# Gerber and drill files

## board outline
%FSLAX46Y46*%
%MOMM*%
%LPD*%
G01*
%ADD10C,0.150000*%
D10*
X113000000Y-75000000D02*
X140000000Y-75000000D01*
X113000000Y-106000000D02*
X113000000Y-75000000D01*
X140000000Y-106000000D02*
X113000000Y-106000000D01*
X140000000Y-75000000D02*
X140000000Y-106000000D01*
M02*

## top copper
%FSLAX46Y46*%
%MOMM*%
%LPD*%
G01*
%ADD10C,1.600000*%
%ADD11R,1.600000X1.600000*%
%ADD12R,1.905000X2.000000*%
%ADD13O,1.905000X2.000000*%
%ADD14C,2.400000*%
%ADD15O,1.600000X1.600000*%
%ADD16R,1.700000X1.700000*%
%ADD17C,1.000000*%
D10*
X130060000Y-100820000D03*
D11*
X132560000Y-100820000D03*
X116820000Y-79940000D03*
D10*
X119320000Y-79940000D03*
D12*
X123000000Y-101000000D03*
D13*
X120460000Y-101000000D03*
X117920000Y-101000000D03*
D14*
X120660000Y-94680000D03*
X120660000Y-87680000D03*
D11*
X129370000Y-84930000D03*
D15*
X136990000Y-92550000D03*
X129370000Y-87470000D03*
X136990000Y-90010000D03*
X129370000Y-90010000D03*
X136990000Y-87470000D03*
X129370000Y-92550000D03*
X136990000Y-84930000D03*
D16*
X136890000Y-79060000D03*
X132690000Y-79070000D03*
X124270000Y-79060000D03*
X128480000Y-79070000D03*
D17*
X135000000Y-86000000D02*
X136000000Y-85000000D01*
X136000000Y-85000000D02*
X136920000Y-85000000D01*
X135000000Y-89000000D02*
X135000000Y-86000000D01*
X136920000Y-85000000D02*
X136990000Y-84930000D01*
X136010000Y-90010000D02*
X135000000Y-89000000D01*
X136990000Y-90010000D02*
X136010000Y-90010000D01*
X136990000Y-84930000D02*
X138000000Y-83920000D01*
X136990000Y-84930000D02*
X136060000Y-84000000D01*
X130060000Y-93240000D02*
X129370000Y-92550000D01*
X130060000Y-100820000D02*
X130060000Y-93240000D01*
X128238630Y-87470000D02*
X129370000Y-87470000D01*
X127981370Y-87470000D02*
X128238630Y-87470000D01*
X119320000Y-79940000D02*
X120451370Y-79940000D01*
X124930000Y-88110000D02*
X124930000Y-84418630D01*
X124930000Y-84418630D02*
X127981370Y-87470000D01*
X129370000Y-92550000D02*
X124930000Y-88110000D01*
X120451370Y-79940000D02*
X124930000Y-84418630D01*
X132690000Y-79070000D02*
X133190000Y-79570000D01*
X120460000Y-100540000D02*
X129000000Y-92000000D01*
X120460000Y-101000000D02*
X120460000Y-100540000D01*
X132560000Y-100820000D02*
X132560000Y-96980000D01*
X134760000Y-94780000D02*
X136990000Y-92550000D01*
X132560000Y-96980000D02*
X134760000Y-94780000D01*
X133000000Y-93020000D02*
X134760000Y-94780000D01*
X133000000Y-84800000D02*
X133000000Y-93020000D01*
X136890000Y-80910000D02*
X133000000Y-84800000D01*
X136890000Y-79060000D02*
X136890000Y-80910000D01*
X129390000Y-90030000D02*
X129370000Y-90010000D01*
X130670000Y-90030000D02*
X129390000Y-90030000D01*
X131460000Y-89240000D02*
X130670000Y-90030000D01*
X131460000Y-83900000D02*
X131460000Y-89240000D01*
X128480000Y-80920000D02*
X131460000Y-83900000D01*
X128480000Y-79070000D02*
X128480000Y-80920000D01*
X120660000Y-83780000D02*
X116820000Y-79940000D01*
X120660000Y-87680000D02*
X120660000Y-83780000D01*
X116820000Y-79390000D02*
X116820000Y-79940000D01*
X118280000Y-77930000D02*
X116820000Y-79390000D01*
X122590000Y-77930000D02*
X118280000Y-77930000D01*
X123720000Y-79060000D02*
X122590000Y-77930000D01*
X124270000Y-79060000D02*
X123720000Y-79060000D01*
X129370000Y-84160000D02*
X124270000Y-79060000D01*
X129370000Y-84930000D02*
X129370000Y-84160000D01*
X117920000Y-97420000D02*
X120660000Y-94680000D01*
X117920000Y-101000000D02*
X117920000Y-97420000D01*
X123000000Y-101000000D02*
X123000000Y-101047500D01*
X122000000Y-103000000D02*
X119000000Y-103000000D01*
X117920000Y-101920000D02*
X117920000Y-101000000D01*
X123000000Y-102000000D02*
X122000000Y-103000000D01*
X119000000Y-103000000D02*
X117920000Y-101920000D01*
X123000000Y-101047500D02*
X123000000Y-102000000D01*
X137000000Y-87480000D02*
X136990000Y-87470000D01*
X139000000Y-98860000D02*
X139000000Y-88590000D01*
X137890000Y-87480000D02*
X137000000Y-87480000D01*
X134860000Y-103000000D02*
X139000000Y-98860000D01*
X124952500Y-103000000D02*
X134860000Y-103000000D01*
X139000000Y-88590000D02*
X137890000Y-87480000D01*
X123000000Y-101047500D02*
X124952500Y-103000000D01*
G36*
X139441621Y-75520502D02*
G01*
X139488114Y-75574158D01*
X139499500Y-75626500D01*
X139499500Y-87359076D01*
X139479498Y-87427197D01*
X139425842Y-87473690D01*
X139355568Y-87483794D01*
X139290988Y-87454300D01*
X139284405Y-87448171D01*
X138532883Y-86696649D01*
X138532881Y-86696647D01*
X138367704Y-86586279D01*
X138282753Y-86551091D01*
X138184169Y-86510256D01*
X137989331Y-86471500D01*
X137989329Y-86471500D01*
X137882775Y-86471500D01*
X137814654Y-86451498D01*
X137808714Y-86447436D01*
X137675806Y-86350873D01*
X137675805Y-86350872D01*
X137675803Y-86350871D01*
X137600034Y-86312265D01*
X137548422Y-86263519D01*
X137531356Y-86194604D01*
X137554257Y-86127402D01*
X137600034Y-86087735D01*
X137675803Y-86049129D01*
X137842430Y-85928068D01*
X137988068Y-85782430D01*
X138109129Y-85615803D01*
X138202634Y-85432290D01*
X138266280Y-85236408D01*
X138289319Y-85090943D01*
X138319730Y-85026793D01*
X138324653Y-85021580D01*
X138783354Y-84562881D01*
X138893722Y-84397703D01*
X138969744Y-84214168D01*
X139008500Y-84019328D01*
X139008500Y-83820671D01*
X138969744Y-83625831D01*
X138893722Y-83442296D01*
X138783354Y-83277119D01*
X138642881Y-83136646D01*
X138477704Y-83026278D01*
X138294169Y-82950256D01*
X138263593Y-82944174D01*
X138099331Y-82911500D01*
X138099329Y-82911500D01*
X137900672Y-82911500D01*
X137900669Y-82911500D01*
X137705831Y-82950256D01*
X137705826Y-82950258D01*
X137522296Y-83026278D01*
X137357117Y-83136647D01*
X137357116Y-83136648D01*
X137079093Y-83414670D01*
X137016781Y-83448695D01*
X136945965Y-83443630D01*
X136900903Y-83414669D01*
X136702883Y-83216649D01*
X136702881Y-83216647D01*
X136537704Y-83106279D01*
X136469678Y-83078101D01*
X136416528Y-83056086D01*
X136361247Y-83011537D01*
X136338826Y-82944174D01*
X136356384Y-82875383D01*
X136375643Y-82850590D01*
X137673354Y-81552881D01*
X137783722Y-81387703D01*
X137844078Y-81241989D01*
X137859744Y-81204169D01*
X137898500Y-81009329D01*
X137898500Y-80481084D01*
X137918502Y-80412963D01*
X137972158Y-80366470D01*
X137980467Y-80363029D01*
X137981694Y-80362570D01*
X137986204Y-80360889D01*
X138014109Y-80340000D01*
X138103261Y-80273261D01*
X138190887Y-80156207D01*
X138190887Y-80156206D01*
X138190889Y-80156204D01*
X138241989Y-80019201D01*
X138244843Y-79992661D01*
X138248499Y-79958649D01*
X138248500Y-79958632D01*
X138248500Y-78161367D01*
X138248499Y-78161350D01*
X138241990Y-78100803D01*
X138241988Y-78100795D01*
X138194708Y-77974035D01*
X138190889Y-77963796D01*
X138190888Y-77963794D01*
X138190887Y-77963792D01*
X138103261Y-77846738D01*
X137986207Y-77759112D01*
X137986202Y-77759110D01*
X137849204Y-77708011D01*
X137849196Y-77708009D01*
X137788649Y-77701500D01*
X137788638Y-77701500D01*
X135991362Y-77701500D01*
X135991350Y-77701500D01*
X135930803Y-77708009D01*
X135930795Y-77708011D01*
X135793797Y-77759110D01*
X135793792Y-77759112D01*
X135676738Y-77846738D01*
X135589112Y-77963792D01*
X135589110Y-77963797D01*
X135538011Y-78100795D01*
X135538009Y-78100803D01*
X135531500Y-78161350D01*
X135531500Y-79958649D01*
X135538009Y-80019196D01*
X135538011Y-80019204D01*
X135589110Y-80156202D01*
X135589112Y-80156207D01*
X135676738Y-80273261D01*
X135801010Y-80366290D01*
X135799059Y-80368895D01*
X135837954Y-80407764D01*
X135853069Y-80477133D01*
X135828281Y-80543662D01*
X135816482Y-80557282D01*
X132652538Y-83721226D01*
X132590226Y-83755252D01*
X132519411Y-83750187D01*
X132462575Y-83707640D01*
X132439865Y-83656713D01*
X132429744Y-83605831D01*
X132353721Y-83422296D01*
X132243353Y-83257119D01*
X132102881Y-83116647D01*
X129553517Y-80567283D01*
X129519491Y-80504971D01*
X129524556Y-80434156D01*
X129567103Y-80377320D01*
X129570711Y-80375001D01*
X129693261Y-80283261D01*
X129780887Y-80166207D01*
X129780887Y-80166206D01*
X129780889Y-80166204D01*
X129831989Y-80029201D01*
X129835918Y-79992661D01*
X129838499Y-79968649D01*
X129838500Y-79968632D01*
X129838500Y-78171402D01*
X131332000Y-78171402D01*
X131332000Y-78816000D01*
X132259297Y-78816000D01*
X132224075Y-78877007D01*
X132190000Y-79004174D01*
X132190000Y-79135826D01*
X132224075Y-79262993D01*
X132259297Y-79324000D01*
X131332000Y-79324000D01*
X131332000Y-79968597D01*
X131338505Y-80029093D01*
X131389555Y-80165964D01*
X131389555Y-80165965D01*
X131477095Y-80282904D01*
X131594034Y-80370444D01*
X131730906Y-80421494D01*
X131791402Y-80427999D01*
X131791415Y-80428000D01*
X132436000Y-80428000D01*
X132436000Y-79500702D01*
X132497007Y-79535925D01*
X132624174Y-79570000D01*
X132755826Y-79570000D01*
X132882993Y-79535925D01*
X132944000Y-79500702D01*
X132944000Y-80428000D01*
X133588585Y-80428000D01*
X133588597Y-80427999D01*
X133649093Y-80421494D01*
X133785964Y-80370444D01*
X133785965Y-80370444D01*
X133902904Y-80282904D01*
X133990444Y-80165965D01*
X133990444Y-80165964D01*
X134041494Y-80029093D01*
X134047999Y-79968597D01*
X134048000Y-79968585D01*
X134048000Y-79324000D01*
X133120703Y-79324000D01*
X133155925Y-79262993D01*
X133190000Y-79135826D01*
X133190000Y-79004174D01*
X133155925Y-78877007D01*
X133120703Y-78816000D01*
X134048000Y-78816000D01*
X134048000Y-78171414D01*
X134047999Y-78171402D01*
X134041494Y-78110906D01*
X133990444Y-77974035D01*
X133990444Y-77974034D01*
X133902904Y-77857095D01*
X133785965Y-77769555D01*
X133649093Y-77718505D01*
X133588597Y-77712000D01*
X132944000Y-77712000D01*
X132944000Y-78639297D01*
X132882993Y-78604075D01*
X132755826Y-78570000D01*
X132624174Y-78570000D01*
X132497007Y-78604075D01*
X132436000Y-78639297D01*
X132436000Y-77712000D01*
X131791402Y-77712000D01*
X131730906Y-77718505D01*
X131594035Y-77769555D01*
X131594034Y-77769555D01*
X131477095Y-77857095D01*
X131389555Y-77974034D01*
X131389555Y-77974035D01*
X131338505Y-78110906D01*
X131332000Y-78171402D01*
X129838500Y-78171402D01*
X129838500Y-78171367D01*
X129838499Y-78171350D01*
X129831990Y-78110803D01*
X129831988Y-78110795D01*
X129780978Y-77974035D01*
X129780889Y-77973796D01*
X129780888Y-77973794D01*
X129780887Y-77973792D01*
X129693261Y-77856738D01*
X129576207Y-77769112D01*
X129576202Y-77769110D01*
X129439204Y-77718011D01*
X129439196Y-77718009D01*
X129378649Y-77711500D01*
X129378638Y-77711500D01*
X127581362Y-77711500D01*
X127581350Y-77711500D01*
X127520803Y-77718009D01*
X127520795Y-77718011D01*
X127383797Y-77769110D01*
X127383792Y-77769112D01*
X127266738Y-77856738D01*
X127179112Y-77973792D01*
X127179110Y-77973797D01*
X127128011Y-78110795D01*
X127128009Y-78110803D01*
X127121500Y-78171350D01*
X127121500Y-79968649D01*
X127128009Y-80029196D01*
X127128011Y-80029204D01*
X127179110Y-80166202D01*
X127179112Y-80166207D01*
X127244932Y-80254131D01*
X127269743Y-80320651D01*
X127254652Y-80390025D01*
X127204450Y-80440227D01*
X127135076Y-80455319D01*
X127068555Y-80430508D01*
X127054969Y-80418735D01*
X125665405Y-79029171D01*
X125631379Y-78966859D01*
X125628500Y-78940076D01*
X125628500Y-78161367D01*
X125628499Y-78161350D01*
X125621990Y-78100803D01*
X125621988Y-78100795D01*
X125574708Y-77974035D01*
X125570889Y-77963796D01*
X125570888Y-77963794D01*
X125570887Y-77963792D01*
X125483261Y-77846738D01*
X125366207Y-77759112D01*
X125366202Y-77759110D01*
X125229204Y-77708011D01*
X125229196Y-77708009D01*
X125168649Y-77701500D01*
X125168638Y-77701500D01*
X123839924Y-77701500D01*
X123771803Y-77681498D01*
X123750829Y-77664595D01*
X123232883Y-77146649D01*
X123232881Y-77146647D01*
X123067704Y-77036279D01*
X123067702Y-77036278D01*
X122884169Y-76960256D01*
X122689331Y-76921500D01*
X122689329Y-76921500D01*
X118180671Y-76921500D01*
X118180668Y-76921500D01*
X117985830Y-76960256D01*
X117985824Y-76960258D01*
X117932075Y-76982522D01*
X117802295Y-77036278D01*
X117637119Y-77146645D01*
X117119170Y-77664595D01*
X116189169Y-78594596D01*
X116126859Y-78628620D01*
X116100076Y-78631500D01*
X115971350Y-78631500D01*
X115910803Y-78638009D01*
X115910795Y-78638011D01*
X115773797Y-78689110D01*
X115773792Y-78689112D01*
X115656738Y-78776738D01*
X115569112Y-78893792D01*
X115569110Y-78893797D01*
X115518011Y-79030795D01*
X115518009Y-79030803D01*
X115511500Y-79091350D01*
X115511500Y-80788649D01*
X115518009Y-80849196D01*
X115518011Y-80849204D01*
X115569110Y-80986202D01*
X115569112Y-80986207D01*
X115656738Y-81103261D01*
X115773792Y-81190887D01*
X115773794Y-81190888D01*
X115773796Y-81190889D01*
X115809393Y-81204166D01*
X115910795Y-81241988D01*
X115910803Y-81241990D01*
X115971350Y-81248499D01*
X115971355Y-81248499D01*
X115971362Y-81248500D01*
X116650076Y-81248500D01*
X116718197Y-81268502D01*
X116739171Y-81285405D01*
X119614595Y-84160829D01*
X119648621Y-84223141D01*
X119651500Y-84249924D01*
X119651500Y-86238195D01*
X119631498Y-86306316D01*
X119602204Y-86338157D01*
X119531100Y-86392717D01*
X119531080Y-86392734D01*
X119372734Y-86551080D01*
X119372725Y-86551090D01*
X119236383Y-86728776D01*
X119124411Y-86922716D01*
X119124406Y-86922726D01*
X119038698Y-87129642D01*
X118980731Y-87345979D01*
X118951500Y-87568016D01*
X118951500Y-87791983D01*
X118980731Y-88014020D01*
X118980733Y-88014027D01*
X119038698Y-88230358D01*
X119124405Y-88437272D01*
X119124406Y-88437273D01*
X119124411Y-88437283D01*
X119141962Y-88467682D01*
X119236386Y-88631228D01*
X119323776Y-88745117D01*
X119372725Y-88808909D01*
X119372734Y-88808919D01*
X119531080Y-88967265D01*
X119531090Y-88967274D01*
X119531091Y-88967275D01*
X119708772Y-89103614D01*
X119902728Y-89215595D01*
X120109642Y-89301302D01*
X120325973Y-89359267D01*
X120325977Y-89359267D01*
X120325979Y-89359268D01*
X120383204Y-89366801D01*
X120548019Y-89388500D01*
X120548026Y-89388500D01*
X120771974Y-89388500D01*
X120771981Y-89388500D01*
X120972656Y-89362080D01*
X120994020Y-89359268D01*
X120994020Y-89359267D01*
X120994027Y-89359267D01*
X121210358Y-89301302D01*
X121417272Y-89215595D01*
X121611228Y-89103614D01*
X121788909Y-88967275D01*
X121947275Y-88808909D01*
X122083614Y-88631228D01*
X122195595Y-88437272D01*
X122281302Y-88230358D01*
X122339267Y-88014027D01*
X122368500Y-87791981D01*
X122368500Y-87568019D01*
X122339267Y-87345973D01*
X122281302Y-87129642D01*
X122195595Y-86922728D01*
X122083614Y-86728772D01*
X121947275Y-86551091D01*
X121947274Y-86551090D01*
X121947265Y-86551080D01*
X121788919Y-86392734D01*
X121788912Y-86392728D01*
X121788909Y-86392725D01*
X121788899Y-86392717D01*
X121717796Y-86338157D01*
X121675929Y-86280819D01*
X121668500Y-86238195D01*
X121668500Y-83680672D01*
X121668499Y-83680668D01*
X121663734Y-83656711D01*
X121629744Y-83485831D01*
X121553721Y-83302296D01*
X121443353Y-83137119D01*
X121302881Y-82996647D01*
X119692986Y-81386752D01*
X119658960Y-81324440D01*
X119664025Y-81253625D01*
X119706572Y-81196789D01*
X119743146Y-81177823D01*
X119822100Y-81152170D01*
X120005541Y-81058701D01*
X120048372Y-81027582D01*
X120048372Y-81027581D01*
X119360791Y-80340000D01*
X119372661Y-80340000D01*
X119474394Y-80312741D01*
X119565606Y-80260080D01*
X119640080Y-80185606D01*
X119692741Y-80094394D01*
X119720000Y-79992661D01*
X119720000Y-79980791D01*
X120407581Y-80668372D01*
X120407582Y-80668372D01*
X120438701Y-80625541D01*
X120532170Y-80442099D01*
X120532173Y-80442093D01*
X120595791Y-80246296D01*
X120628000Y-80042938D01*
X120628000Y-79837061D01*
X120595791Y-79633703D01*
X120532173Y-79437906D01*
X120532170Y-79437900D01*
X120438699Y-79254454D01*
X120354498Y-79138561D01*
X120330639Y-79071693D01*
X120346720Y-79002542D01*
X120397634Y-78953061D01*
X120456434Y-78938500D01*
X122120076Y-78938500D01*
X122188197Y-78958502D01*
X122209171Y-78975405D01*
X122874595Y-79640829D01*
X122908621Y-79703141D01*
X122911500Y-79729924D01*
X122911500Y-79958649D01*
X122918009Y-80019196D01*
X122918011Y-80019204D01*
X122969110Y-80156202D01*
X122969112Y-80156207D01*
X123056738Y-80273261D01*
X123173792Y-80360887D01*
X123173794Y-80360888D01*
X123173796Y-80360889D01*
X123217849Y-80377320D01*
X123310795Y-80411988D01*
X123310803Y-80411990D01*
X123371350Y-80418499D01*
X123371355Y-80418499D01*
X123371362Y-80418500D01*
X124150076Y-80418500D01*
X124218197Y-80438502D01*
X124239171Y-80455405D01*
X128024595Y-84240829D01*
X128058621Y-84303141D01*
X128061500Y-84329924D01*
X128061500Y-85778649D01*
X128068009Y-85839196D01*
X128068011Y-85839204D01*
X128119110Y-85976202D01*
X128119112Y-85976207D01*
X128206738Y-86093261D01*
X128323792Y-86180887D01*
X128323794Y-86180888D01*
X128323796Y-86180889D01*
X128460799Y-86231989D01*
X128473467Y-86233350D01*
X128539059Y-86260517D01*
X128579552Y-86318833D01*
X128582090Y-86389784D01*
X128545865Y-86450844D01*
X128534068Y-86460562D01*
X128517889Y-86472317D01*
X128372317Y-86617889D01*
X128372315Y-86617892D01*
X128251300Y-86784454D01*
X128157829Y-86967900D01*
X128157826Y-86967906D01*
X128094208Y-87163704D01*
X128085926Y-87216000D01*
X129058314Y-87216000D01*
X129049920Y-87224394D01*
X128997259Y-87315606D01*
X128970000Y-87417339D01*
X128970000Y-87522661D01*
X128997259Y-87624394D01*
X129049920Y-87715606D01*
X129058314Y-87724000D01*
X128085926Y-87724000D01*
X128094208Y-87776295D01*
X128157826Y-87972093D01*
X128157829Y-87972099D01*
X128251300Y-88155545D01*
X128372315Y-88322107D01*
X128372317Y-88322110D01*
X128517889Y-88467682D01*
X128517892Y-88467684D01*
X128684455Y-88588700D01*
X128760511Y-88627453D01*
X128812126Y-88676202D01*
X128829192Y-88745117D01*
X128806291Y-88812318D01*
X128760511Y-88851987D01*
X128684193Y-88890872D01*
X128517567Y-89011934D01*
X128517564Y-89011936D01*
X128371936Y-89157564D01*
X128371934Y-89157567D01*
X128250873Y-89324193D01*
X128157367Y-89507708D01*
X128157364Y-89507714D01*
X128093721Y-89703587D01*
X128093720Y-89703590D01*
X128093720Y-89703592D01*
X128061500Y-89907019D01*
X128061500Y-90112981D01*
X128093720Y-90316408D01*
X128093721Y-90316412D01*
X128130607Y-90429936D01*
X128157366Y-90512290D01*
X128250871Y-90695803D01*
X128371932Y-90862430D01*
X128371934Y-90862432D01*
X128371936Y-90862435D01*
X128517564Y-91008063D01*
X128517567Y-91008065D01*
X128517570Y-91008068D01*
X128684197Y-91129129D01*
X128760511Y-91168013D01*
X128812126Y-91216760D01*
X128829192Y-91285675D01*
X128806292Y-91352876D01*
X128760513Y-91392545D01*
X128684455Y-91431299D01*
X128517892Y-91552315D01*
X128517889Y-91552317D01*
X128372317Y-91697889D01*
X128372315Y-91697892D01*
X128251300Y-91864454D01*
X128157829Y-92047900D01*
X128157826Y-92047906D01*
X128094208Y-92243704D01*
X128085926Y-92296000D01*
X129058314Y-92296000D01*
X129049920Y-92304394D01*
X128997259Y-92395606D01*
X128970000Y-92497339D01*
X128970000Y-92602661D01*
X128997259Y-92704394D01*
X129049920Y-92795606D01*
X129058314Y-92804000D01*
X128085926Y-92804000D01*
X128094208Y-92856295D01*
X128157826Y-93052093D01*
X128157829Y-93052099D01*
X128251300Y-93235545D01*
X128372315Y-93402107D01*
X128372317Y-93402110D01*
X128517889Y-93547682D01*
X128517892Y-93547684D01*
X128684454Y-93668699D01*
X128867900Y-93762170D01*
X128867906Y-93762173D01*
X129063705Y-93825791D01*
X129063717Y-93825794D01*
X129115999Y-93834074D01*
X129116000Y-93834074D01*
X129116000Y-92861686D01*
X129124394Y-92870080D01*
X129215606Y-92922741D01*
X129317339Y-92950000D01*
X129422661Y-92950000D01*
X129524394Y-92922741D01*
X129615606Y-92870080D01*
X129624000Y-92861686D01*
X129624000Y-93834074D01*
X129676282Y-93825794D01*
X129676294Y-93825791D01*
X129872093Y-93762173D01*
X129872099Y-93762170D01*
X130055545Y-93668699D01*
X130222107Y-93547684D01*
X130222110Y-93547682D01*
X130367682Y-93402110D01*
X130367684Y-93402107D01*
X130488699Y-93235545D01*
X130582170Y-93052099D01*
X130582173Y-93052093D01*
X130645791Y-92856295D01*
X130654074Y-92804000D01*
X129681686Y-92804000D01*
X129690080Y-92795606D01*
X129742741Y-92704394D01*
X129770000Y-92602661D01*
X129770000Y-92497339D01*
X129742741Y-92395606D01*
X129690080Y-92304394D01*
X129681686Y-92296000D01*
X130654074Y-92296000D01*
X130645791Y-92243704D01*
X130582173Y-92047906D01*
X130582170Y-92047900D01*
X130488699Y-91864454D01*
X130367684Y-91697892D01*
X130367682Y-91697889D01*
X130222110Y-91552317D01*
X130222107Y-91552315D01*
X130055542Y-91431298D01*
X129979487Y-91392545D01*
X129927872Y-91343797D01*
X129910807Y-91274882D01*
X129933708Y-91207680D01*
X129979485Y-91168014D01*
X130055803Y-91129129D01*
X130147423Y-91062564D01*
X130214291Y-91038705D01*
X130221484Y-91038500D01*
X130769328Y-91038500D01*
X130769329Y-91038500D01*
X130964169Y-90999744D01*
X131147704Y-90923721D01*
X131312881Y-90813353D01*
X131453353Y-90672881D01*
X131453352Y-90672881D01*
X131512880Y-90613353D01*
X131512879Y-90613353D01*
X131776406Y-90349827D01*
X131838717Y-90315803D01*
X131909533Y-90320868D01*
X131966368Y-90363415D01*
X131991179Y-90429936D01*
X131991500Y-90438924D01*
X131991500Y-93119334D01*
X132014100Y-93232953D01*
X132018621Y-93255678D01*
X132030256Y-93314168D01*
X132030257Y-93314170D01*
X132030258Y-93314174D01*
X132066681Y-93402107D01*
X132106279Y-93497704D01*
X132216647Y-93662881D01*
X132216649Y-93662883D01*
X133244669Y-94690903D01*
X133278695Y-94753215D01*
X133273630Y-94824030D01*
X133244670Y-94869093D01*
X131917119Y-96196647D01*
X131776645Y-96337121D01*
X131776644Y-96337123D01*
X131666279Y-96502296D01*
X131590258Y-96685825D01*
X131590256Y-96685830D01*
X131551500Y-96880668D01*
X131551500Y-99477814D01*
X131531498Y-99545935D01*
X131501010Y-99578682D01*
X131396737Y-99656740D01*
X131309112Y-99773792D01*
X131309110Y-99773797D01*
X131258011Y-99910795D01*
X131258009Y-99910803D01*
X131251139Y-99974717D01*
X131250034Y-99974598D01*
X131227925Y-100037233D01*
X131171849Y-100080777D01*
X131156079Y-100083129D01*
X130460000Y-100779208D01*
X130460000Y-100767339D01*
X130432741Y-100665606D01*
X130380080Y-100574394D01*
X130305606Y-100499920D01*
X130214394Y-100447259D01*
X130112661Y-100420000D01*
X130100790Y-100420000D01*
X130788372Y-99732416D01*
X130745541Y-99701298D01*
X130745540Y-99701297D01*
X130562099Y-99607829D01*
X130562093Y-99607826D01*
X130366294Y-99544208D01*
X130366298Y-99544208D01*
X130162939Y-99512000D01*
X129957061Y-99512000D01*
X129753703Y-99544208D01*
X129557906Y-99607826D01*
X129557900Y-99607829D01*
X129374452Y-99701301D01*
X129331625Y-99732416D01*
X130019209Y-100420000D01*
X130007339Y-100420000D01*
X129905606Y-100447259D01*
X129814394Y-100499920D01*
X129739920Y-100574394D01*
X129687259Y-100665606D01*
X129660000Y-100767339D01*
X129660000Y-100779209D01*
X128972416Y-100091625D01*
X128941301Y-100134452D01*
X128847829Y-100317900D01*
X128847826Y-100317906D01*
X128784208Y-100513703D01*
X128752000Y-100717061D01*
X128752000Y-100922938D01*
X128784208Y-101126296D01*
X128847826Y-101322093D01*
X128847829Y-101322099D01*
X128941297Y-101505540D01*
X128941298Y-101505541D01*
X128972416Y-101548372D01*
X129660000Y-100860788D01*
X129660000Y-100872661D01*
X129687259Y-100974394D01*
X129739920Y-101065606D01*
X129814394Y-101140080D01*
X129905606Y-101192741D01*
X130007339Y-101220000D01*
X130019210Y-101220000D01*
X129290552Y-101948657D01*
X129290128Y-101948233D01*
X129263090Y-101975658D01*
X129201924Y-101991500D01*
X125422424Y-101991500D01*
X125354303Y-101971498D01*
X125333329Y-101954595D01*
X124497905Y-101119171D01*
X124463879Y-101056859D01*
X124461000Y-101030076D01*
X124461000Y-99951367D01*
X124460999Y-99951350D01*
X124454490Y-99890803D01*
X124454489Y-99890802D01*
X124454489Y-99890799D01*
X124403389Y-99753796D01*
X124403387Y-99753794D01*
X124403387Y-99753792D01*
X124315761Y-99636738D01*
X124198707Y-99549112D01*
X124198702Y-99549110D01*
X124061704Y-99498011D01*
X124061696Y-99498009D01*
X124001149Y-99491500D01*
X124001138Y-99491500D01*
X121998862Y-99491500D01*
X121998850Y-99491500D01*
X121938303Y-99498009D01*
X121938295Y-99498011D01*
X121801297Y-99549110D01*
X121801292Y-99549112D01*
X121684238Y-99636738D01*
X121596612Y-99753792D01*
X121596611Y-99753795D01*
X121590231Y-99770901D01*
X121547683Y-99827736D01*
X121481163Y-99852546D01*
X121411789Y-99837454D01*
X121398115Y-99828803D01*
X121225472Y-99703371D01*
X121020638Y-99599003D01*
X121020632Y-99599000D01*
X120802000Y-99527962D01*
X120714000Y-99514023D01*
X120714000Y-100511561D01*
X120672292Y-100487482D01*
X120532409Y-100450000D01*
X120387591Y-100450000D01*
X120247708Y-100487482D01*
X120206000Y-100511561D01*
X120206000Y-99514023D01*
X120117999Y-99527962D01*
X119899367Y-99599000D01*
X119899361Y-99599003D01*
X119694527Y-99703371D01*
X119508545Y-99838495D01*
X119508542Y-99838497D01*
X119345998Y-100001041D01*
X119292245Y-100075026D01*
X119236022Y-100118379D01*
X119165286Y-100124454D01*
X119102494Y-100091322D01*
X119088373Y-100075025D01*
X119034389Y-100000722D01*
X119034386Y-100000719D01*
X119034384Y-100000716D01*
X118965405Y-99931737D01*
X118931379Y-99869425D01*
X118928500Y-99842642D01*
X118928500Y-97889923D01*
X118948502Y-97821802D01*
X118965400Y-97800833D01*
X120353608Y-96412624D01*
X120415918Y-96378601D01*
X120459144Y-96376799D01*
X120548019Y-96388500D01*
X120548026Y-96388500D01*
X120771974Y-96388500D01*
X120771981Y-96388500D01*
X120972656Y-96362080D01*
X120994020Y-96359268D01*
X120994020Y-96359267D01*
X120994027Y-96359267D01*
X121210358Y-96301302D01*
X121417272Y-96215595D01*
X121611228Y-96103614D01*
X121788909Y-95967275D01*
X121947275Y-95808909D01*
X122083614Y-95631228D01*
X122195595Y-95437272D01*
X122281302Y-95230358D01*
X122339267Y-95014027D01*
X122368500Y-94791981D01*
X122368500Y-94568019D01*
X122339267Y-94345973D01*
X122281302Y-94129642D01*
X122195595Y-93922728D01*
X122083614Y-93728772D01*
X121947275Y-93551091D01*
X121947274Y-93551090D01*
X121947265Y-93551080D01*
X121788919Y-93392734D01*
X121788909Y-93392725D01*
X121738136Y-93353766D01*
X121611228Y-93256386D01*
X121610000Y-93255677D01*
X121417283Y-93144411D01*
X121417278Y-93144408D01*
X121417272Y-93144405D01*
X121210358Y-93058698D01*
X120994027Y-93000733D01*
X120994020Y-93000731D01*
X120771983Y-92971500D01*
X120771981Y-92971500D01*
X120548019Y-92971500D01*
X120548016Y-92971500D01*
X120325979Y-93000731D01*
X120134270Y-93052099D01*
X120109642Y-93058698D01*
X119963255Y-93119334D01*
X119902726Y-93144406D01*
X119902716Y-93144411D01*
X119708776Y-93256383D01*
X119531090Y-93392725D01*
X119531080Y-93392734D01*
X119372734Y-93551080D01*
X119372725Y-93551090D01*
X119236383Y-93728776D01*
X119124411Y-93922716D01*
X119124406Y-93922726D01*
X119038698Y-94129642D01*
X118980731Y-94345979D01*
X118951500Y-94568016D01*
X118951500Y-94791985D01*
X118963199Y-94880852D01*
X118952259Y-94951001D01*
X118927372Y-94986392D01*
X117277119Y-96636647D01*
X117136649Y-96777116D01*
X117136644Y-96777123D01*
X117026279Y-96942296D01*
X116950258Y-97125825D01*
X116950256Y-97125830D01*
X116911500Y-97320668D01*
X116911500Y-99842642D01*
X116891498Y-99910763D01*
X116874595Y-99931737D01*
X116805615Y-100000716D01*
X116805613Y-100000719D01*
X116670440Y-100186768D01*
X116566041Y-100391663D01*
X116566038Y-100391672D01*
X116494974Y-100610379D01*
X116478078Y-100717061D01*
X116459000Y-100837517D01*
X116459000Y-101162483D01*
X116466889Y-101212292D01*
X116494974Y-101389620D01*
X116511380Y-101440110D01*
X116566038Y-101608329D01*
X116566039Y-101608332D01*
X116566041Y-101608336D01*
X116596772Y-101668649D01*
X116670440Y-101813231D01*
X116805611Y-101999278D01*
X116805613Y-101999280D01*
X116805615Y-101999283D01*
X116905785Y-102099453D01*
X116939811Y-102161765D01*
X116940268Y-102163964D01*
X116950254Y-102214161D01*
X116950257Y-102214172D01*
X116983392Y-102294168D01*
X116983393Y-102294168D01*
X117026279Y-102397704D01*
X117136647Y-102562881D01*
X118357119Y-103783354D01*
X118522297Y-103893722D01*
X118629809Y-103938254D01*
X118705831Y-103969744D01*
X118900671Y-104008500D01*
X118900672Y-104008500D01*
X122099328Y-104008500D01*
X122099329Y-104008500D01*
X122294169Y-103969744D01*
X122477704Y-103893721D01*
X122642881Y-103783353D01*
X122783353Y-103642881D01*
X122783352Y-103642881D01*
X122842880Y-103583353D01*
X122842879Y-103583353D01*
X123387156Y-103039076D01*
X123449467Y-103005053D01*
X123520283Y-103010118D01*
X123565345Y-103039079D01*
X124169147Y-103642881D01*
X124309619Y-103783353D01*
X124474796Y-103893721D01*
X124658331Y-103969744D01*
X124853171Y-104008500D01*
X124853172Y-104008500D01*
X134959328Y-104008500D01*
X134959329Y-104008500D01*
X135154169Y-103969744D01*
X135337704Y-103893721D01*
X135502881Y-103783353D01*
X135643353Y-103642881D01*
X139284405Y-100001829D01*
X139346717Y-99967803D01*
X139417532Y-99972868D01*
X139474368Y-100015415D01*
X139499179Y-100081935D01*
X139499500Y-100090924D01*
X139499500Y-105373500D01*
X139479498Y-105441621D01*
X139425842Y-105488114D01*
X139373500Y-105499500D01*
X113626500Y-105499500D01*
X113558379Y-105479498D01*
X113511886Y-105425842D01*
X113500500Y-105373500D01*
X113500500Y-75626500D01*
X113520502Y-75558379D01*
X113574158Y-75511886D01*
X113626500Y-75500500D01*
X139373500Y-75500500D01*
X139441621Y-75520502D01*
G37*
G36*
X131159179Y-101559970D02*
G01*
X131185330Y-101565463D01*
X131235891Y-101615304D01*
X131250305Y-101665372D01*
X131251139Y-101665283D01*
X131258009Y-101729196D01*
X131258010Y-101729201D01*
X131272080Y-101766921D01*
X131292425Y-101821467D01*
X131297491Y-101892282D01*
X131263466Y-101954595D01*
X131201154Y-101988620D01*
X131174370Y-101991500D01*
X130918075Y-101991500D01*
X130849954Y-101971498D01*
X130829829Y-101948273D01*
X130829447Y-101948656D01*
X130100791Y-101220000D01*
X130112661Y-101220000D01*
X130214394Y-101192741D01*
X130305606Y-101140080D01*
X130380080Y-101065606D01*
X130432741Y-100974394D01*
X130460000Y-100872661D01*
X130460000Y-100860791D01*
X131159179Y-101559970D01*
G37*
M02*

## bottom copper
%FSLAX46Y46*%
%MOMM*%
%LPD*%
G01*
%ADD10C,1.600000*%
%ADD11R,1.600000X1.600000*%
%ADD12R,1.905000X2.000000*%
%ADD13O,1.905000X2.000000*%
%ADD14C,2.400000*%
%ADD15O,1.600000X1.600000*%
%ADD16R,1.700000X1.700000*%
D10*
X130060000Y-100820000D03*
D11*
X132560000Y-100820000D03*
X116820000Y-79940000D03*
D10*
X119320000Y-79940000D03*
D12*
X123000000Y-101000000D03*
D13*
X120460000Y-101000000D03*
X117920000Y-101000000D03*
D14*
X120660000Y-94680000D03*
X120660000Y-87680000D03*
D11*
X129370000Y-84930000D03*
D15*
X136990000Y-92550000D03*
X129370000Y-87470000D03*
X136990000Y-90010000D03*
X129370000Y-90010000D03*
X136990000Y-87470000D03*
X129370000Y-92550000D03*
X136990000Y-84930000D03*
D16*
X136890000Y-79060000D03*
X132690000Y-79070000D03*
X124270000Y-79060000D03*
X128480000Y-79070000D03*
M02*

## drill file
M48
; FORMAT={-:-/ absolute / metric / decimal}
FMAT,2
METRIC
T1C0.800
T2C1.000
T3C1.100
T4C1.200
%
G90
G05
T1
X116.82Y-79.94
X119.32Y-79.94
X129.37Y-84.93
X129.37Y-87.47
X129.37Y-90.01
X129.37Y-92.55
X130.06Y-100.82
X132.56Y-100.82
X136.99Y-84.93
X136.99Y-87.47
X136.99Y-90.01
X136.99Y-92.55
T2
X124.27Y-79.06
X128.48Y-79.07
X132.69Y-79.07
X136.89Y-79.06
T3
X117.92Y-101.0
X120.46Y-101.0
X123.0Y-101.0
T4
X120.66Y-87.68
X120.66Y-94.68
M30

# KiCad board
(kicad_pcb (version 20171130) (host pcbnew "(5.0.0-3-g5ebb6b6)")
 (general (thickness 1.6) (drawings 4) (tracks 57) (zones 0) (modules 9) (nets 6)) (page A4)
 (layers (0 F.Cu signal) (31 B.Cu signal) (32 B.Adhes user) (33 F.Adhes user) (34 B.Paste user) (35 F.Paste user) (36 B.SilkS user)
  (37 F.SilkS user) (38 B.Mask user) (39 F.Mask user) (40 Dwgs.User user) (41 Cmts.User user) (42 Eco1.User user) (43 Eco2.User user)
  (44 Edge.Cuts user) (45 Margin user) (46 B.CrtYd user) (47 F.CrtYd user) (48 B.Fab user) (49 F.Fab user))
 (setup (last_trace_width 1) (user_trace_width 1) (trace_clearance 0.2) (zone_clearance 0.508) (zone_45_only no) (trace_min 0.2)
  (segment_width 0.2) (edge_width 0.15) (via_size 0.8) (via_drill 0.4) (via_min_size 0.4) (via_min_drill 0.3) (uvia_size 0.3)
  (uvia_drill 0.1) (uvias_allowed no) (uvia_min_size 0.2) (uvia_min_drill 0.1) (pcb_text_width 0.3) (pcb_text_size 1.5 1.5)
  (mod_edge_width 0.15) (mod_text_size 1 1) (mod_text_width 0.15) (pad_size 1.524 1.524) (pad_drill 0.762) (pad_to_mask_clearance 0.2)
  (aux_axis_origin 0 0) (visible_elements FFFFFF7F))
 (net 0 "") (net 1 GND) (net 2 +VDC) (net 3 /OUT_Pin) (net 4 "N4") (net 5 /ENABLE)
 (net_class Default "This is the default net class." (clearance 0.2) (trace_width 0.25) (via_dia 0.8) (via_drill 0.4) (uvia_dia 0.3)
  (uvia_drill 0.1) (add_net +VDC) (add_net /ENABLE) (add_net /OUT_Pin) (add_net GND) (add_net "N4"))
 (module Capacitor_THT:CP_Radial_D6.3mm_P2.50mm (layer F.Cu) (at 132.56 100.82 180)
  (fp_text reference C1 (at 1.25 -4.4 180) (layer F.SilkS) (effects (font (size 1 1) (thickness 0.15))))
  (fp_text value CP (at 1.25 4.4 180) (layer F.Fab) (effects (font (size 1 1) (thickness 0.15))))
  (pad 2 thru_hole circle (at 2.5 0 180) (size 1.6 1.6) (drill 0.8) (layers *.Cu *.Mask) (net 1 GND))
  (pad 1 thru_hole rect (at 0 0 180) (size 1.6 1.6) (drill 0.8) (layers *.Cu *.Mask) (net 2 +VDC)))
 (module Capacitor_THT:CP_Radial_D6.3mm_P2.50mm (layer F.Cu) (at 116.82 79.94)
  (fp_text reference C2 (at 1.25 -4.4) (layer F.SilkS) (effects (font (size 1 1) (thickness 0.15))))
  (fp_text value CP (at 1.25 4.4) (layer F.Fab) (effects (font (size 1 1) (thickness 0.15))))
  (pad 1 thru_hole rect (at 0 0) (size 1.6 1.6) (drill 0.8) (layers *.Cu *.Mask) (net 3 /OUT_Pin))
  (pad 2 thru_hole circle (at 2.5 0) (size 1.6 1.6) (drill 0.8) (layers *.Cu *.Mask) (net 1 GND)))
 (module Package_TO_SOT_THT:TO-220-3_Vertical (layer F.Cu) (at 123 101 180)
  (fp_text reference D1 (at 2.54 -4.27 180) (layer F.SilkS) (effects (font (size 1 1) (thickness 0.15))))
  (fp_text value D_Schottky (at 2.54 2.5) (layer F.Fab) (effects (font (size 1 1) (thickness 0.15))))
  (pad 1 thru_hole rect (at 0 0 180) (size 1.905 2) (drill 1.1) (layers *.Cu *.Mask) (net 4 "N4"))
  (pad 2 thru_hole oval (at 2.54 0 180) (size 1.905 2) (drill 1.1) (layers *.Cu *.Mask) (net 1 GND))
  (pad 3 thru_hole oval (at 5.08 0 180) (size 1.905 2) (drill 1.1) (layers *.Cu *.Mask) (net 4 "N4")))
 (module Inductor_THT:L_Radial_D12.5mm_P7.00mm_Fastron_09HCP (layer F.Cu) (at 120.66 94.68 90)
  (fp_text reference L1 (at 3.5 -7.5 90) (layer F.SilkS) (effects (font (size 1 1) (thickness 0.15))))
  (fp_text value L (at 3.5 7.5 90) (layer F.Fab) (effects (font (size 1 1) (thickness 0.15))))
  (pad 1 thru_hole circle (at 0 0 90) (size 2.4 2.4) (drill 1.2) (layers *.Cu *.Mask) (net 4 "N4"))
  (pad 2 thru_hole circle (at 7 0 90) (size 2.4 2.4) (drill 1.2) (layers *.Cu *.Mask) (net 3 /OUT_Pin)))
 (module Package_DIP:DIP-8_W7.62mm (layer F.Cu) (at 129.37 84.93)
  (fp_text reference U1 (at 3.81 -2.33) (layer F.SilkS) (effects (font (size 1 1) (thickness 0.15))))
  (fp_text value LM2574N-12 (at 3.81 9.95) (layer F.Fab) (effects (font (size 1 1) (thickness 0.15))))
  (pad 1 thru_hole rect (at 0 0) (size 1.6 1.6) (drill 0.8) (layers *.Cu *.Mask) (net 3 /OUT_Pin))
  (pad 5 thru_hole oval (at 7.62 7.62) (size 1.6 1.6) (drill 0.8) (layers *.Cu *.Mask) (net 2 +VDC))
  (pad 2 thru_hole oval (at 0 2.54) (size 1.6 1.6) (drill 0.8) (layers *.Cu *.Mask) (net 1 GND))
  (pad 6 thru_hole oval (at 7.62 5.08) (size 1.6 1.6) (drill 0.8) (layers *.Cu *.Mask))
  (pad 3 thru_hole oval (at 0 5.08) (size 1.6 1.6) (drill 0.8) (layers *.Cu *.Mask) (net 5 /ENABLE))
  (pad 7 thru_hole oval (at 7.62 2.54) (size 1.6 1.6) (drill 0.8) (layers *.Cu *.Mask) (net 4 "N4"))
  (pad 4 thru_hole oval (at 0 7.62) (size 1.6 1.6) (drill 0.8) (layers *.Cu *.Mask) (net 1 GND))
  (pad 8 thru_hole oval (at 7.62 0) (size 1.6 1.6) (drill 0.8) (layers *.Cu *.Mask)))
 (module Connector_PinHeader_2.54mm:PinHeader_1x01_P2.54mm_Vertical (layer F.Cu) (at 136.89 79.06)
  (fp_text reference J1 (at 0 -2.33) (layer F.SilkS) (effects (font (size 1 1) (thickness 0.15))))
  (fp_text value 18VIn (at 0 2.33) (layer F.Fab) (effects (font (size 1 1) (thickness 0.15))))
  (pad 1 thru_hole rect (at 0 0) (size 1.7 1.7) (drill 1) (layers *.Cu *.Mask) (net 2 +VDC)))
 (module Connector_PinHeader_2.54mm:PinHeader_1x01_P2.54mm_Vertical (layer F.Cu) (at 132.69 79.07 180)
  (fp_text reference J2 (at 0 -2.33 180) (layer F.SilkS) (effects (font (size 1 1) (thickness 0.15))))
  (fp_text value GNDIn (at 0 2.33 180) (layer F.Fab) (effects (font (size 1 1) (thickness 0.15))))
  (pad 1 thru_hole rect (at 0 0 180) (size 1.7 1.7) (drill 1) (layers *.Cu *.Mask) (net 1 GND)))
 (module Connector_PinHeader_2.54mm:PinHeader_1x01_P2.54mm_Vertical (layer F.Cu) (at 124.27 79.06 180)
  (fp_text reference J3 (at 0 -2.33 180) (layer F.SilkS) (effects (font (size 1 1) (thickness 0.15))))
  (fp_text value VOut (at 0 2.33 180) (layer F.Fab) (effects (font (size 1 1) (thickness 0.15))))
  (pad 1 thru_hole rect (at 0 0 180) (size 1.7 1.7) (drill 1) (layers *.Cu *.Mask) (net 3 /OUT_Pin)))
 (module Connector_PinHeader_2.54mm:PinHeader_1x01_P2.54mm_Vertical (layer F.Cu) (at 128.48 79.07 180)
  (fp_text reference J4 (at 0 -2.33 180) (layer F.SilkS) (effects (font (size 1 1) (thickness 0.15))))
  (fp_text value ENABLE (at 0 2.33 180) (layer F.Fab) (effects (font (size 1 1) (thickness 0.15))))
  (pad 1 thru_hole rect (at 0 0 180) (size 1.7 1.7) (drill 1) (layers *.Cu *.Mask) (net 5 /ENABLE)))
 (gr_line (start 113 75) (end 140 75) (layer Edge.Cuts) (width 0.15))
 (gr_line (start 113 106) (end 113 75) (layer Edge.Cuts) (width 0.15))
 (gr_line (start 140 106) (end 113 106) (layer Edge.Cuts) (width 0.15))
 (gr_line (start 140 75) (end 140 106) (layer Edge.Cuts) (width 0.15))
 (segment (start 135 86) (end 136 85) (width 1) (layer F.Cu) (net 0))
 (segment (start 136 85) (end 136.92 85) (width 1) (layer F.Cu) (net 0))
 (segment (start 135 89) (end 135 86) (width 1) (layer F.Cu) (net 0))
 (segment (start 136.92 85) (end 136.99 84.93) (width 1) (layer F.Cu) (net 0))
 (segment (start 136.01 90.01) (end 135 89) (width 1) (layer F.Cu) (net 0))
 (segment (start 136.99 90.01) (end 136.01 90.01) (width 1) (layer F.Cu) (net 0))
 (segment (start 136.99 84.93) (end 138 83.92) (width 1) (layer F.Cu) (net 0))
 (segment (start 136.99 84.93) (end 136.06 84) (width 1) (layer F.Cu) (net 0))
 (segment (start 130.06 93.24) (end 129.37 92.55) (width 1) (layer F.Cu) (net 1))
 (segment (start 130.06 100.82) (end 130.06 93.24) (width 1) (layer F.Cu) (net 1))
 (segment (start 128.23863 87.47) (end 129.37 87.47) (width 1) (layer F.Cu) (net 1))
 (segment (start 127.98137 87.47) (end 128.23863 87.47) (width 1) (layer F.Cu) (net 1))
 (segment (start 119.32 79.94) (end 120.45137 79.94) (width 1) (layer F.Cu) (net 1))
 (segment (start 124.93 88.11) (end 124.93 84.41863) (width 1) (layer F.Cu) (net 1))
 (segment (start 124.93 84.41863) (end 127.98137 87.47) (width 1) (layer F.Cu) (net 1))
 (segment (start 129.37 92.55) (end 124.93 88.11) (width 1) (layer F.Cu) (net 1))
 (segment (start 120.45137 79.94) (end 124.93 84.41863) (width 1) (layer F.Cu) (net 1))
 (segment (start 132.69 79.07) (end 133.19 79.57) (width 1) (layer F.Cu) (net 1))
 (segment (start 120.46 100.54) (end 129 92) (width 1) (layer F.Cu) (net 1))
 (segment (start 120.46 101) (end 120.46 100.54) (width 1) (layer F.Cu) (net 1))
 (segment (start 132.56 100.82) (end 132.56 96.98) (width 1) (layer F.Cu) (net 2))
 (segment (start 134.76 94.78) (end 136.99 92.55) (width 1) (layer F.Cu) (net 2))
 (segment (start 132.56 96.98) (end 134.76 94.78) (width 1) (layer F.Cu) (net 2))
 (segment (start 133 93.02) (end 134.76 94.78) (width 1) (layer F.Cu) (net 2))
 (segment (start 133 84.8) (end 133 93.02) (width 1) (layer F.Cu) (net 2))
 (segment (start 136.89 80.91) (end 133 84.8) (width 1) (layer F.Cu) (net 2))
 (segment (start 136.89 79.06) (end 136.89 80.91) (width 1) (layer F.Cu) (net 2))
 (segment (start 129.39 90.03) (end 129.37 90.01) (width 1) (layer F.Cu) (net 5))
 (segment (start 130.67 90.03) (end 129.39 90.03) (width 1) (layer F.Cu) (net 5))
 (segment (start 131.46 89.24) (end 130.67 90.03) (width 1) (layer F.Cu) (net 5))
 (segment (start 131.46 83.9) (end 131.46 89.24) (width 1) (layer F.Cu) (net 5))
 (segment (start 128.48 80.92) (end 131.46 83.9) (width 1) (layer F.Cu) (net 5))
 (segment (start 128.48 79.07) (end 128.48 80.92) (width 1) (layer F.Cu) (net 5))
 (segment (start 120.66 83.78) (end 116.82 79.94) (width 1) (layer F.Cu) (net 3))
 (segment (start 120.66 87.68) (end 120.66 83.78) (width 1) (layer F.Cu) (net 3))
 (segment (start 116.82 79.39) (end 116.82 79.94) (width 1) (layer F.Cu) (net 3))
 (segment (start 118.28 77.93) (end 116.82 79.39) (width 1) (layer F.Cu) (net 3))
 (segment (start 122.59 77.93) (end 118.28 77.93) (width 1) (layer F.Cu) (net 3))
 (segment (start 123.72 79.06) (end 122.59 77.93) (width 1) (layer F.Cu) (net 3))
 (segment (start 124.27 79.06) (end 123.72 79.06) (width 1) (layer F.Cu) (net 3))
 (segment (start 129.37 84.16) (end 124.27 79.06) (width 1) (layer F.Cu) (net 3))
 (segment (start 129.37 84.93) (end 129.37 84.16) (width 1) (layer F.Cu) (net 3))
 (segment (start 117.92 97.42) (end 120.66 94.68) (width 1) (layer F.Cu) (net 4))
 (segment (start 117.92 101) (end 117.92 97.42) (width 1) (layer F.Cu) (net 4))
 (segment (start 123 101) (end 123 101.0475) (width 1) (layer F.Cu) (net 4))
 (segment (start 122 103) (end 119 103) (width 1) (layer F.Cu) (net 4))
 (segment (start 117.92 101.92) (end 117.92 101) (width 1) (layer F.Cu) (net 4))
 (segment (start 123 102) (end 122 103) (width 1) (layer F.Cu) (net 4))
 (segment (start 119 103) (end 117.92 101.92) (width 1) (layer F.Cu) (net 4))
 (segment (start 123 101.0475) (end 123 102) (width 1) (layer F.Cu) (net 4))
 (segment (start 137 87.48) (end 136.99 87.47) (width 1) (layer F.Cu) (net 4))
 (segment (start 139 98.86) (end 139 88.59) (width 1) (layer F.Cu) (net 4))
 (segment (start 137.89 87.48) (end 137 87.48) (width 1) (layer F.Cu) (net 4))
 (segment (start 134.86 103) (end 139 98.86) (width 1) (layer F.Cu) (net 4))
 (segment (start 124.9525 103) (end 134.86 103) (width 1) (layer F.Cu) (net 4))
 (segment (start 139 88.59) (end 137.89 87.48) (width 1) (layer F.Cu) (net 4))
 (segment (start 123 101.0475) (end 124.9525 103) (width 1) (layer F.Cu) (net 4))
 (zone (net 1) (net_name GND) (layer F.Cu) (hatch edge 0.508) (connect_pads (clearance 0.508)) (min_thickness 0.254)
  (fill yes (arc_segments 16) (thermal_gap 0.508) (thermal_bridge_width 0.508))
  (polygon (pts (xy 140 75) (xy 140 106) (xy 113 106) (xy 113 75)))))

